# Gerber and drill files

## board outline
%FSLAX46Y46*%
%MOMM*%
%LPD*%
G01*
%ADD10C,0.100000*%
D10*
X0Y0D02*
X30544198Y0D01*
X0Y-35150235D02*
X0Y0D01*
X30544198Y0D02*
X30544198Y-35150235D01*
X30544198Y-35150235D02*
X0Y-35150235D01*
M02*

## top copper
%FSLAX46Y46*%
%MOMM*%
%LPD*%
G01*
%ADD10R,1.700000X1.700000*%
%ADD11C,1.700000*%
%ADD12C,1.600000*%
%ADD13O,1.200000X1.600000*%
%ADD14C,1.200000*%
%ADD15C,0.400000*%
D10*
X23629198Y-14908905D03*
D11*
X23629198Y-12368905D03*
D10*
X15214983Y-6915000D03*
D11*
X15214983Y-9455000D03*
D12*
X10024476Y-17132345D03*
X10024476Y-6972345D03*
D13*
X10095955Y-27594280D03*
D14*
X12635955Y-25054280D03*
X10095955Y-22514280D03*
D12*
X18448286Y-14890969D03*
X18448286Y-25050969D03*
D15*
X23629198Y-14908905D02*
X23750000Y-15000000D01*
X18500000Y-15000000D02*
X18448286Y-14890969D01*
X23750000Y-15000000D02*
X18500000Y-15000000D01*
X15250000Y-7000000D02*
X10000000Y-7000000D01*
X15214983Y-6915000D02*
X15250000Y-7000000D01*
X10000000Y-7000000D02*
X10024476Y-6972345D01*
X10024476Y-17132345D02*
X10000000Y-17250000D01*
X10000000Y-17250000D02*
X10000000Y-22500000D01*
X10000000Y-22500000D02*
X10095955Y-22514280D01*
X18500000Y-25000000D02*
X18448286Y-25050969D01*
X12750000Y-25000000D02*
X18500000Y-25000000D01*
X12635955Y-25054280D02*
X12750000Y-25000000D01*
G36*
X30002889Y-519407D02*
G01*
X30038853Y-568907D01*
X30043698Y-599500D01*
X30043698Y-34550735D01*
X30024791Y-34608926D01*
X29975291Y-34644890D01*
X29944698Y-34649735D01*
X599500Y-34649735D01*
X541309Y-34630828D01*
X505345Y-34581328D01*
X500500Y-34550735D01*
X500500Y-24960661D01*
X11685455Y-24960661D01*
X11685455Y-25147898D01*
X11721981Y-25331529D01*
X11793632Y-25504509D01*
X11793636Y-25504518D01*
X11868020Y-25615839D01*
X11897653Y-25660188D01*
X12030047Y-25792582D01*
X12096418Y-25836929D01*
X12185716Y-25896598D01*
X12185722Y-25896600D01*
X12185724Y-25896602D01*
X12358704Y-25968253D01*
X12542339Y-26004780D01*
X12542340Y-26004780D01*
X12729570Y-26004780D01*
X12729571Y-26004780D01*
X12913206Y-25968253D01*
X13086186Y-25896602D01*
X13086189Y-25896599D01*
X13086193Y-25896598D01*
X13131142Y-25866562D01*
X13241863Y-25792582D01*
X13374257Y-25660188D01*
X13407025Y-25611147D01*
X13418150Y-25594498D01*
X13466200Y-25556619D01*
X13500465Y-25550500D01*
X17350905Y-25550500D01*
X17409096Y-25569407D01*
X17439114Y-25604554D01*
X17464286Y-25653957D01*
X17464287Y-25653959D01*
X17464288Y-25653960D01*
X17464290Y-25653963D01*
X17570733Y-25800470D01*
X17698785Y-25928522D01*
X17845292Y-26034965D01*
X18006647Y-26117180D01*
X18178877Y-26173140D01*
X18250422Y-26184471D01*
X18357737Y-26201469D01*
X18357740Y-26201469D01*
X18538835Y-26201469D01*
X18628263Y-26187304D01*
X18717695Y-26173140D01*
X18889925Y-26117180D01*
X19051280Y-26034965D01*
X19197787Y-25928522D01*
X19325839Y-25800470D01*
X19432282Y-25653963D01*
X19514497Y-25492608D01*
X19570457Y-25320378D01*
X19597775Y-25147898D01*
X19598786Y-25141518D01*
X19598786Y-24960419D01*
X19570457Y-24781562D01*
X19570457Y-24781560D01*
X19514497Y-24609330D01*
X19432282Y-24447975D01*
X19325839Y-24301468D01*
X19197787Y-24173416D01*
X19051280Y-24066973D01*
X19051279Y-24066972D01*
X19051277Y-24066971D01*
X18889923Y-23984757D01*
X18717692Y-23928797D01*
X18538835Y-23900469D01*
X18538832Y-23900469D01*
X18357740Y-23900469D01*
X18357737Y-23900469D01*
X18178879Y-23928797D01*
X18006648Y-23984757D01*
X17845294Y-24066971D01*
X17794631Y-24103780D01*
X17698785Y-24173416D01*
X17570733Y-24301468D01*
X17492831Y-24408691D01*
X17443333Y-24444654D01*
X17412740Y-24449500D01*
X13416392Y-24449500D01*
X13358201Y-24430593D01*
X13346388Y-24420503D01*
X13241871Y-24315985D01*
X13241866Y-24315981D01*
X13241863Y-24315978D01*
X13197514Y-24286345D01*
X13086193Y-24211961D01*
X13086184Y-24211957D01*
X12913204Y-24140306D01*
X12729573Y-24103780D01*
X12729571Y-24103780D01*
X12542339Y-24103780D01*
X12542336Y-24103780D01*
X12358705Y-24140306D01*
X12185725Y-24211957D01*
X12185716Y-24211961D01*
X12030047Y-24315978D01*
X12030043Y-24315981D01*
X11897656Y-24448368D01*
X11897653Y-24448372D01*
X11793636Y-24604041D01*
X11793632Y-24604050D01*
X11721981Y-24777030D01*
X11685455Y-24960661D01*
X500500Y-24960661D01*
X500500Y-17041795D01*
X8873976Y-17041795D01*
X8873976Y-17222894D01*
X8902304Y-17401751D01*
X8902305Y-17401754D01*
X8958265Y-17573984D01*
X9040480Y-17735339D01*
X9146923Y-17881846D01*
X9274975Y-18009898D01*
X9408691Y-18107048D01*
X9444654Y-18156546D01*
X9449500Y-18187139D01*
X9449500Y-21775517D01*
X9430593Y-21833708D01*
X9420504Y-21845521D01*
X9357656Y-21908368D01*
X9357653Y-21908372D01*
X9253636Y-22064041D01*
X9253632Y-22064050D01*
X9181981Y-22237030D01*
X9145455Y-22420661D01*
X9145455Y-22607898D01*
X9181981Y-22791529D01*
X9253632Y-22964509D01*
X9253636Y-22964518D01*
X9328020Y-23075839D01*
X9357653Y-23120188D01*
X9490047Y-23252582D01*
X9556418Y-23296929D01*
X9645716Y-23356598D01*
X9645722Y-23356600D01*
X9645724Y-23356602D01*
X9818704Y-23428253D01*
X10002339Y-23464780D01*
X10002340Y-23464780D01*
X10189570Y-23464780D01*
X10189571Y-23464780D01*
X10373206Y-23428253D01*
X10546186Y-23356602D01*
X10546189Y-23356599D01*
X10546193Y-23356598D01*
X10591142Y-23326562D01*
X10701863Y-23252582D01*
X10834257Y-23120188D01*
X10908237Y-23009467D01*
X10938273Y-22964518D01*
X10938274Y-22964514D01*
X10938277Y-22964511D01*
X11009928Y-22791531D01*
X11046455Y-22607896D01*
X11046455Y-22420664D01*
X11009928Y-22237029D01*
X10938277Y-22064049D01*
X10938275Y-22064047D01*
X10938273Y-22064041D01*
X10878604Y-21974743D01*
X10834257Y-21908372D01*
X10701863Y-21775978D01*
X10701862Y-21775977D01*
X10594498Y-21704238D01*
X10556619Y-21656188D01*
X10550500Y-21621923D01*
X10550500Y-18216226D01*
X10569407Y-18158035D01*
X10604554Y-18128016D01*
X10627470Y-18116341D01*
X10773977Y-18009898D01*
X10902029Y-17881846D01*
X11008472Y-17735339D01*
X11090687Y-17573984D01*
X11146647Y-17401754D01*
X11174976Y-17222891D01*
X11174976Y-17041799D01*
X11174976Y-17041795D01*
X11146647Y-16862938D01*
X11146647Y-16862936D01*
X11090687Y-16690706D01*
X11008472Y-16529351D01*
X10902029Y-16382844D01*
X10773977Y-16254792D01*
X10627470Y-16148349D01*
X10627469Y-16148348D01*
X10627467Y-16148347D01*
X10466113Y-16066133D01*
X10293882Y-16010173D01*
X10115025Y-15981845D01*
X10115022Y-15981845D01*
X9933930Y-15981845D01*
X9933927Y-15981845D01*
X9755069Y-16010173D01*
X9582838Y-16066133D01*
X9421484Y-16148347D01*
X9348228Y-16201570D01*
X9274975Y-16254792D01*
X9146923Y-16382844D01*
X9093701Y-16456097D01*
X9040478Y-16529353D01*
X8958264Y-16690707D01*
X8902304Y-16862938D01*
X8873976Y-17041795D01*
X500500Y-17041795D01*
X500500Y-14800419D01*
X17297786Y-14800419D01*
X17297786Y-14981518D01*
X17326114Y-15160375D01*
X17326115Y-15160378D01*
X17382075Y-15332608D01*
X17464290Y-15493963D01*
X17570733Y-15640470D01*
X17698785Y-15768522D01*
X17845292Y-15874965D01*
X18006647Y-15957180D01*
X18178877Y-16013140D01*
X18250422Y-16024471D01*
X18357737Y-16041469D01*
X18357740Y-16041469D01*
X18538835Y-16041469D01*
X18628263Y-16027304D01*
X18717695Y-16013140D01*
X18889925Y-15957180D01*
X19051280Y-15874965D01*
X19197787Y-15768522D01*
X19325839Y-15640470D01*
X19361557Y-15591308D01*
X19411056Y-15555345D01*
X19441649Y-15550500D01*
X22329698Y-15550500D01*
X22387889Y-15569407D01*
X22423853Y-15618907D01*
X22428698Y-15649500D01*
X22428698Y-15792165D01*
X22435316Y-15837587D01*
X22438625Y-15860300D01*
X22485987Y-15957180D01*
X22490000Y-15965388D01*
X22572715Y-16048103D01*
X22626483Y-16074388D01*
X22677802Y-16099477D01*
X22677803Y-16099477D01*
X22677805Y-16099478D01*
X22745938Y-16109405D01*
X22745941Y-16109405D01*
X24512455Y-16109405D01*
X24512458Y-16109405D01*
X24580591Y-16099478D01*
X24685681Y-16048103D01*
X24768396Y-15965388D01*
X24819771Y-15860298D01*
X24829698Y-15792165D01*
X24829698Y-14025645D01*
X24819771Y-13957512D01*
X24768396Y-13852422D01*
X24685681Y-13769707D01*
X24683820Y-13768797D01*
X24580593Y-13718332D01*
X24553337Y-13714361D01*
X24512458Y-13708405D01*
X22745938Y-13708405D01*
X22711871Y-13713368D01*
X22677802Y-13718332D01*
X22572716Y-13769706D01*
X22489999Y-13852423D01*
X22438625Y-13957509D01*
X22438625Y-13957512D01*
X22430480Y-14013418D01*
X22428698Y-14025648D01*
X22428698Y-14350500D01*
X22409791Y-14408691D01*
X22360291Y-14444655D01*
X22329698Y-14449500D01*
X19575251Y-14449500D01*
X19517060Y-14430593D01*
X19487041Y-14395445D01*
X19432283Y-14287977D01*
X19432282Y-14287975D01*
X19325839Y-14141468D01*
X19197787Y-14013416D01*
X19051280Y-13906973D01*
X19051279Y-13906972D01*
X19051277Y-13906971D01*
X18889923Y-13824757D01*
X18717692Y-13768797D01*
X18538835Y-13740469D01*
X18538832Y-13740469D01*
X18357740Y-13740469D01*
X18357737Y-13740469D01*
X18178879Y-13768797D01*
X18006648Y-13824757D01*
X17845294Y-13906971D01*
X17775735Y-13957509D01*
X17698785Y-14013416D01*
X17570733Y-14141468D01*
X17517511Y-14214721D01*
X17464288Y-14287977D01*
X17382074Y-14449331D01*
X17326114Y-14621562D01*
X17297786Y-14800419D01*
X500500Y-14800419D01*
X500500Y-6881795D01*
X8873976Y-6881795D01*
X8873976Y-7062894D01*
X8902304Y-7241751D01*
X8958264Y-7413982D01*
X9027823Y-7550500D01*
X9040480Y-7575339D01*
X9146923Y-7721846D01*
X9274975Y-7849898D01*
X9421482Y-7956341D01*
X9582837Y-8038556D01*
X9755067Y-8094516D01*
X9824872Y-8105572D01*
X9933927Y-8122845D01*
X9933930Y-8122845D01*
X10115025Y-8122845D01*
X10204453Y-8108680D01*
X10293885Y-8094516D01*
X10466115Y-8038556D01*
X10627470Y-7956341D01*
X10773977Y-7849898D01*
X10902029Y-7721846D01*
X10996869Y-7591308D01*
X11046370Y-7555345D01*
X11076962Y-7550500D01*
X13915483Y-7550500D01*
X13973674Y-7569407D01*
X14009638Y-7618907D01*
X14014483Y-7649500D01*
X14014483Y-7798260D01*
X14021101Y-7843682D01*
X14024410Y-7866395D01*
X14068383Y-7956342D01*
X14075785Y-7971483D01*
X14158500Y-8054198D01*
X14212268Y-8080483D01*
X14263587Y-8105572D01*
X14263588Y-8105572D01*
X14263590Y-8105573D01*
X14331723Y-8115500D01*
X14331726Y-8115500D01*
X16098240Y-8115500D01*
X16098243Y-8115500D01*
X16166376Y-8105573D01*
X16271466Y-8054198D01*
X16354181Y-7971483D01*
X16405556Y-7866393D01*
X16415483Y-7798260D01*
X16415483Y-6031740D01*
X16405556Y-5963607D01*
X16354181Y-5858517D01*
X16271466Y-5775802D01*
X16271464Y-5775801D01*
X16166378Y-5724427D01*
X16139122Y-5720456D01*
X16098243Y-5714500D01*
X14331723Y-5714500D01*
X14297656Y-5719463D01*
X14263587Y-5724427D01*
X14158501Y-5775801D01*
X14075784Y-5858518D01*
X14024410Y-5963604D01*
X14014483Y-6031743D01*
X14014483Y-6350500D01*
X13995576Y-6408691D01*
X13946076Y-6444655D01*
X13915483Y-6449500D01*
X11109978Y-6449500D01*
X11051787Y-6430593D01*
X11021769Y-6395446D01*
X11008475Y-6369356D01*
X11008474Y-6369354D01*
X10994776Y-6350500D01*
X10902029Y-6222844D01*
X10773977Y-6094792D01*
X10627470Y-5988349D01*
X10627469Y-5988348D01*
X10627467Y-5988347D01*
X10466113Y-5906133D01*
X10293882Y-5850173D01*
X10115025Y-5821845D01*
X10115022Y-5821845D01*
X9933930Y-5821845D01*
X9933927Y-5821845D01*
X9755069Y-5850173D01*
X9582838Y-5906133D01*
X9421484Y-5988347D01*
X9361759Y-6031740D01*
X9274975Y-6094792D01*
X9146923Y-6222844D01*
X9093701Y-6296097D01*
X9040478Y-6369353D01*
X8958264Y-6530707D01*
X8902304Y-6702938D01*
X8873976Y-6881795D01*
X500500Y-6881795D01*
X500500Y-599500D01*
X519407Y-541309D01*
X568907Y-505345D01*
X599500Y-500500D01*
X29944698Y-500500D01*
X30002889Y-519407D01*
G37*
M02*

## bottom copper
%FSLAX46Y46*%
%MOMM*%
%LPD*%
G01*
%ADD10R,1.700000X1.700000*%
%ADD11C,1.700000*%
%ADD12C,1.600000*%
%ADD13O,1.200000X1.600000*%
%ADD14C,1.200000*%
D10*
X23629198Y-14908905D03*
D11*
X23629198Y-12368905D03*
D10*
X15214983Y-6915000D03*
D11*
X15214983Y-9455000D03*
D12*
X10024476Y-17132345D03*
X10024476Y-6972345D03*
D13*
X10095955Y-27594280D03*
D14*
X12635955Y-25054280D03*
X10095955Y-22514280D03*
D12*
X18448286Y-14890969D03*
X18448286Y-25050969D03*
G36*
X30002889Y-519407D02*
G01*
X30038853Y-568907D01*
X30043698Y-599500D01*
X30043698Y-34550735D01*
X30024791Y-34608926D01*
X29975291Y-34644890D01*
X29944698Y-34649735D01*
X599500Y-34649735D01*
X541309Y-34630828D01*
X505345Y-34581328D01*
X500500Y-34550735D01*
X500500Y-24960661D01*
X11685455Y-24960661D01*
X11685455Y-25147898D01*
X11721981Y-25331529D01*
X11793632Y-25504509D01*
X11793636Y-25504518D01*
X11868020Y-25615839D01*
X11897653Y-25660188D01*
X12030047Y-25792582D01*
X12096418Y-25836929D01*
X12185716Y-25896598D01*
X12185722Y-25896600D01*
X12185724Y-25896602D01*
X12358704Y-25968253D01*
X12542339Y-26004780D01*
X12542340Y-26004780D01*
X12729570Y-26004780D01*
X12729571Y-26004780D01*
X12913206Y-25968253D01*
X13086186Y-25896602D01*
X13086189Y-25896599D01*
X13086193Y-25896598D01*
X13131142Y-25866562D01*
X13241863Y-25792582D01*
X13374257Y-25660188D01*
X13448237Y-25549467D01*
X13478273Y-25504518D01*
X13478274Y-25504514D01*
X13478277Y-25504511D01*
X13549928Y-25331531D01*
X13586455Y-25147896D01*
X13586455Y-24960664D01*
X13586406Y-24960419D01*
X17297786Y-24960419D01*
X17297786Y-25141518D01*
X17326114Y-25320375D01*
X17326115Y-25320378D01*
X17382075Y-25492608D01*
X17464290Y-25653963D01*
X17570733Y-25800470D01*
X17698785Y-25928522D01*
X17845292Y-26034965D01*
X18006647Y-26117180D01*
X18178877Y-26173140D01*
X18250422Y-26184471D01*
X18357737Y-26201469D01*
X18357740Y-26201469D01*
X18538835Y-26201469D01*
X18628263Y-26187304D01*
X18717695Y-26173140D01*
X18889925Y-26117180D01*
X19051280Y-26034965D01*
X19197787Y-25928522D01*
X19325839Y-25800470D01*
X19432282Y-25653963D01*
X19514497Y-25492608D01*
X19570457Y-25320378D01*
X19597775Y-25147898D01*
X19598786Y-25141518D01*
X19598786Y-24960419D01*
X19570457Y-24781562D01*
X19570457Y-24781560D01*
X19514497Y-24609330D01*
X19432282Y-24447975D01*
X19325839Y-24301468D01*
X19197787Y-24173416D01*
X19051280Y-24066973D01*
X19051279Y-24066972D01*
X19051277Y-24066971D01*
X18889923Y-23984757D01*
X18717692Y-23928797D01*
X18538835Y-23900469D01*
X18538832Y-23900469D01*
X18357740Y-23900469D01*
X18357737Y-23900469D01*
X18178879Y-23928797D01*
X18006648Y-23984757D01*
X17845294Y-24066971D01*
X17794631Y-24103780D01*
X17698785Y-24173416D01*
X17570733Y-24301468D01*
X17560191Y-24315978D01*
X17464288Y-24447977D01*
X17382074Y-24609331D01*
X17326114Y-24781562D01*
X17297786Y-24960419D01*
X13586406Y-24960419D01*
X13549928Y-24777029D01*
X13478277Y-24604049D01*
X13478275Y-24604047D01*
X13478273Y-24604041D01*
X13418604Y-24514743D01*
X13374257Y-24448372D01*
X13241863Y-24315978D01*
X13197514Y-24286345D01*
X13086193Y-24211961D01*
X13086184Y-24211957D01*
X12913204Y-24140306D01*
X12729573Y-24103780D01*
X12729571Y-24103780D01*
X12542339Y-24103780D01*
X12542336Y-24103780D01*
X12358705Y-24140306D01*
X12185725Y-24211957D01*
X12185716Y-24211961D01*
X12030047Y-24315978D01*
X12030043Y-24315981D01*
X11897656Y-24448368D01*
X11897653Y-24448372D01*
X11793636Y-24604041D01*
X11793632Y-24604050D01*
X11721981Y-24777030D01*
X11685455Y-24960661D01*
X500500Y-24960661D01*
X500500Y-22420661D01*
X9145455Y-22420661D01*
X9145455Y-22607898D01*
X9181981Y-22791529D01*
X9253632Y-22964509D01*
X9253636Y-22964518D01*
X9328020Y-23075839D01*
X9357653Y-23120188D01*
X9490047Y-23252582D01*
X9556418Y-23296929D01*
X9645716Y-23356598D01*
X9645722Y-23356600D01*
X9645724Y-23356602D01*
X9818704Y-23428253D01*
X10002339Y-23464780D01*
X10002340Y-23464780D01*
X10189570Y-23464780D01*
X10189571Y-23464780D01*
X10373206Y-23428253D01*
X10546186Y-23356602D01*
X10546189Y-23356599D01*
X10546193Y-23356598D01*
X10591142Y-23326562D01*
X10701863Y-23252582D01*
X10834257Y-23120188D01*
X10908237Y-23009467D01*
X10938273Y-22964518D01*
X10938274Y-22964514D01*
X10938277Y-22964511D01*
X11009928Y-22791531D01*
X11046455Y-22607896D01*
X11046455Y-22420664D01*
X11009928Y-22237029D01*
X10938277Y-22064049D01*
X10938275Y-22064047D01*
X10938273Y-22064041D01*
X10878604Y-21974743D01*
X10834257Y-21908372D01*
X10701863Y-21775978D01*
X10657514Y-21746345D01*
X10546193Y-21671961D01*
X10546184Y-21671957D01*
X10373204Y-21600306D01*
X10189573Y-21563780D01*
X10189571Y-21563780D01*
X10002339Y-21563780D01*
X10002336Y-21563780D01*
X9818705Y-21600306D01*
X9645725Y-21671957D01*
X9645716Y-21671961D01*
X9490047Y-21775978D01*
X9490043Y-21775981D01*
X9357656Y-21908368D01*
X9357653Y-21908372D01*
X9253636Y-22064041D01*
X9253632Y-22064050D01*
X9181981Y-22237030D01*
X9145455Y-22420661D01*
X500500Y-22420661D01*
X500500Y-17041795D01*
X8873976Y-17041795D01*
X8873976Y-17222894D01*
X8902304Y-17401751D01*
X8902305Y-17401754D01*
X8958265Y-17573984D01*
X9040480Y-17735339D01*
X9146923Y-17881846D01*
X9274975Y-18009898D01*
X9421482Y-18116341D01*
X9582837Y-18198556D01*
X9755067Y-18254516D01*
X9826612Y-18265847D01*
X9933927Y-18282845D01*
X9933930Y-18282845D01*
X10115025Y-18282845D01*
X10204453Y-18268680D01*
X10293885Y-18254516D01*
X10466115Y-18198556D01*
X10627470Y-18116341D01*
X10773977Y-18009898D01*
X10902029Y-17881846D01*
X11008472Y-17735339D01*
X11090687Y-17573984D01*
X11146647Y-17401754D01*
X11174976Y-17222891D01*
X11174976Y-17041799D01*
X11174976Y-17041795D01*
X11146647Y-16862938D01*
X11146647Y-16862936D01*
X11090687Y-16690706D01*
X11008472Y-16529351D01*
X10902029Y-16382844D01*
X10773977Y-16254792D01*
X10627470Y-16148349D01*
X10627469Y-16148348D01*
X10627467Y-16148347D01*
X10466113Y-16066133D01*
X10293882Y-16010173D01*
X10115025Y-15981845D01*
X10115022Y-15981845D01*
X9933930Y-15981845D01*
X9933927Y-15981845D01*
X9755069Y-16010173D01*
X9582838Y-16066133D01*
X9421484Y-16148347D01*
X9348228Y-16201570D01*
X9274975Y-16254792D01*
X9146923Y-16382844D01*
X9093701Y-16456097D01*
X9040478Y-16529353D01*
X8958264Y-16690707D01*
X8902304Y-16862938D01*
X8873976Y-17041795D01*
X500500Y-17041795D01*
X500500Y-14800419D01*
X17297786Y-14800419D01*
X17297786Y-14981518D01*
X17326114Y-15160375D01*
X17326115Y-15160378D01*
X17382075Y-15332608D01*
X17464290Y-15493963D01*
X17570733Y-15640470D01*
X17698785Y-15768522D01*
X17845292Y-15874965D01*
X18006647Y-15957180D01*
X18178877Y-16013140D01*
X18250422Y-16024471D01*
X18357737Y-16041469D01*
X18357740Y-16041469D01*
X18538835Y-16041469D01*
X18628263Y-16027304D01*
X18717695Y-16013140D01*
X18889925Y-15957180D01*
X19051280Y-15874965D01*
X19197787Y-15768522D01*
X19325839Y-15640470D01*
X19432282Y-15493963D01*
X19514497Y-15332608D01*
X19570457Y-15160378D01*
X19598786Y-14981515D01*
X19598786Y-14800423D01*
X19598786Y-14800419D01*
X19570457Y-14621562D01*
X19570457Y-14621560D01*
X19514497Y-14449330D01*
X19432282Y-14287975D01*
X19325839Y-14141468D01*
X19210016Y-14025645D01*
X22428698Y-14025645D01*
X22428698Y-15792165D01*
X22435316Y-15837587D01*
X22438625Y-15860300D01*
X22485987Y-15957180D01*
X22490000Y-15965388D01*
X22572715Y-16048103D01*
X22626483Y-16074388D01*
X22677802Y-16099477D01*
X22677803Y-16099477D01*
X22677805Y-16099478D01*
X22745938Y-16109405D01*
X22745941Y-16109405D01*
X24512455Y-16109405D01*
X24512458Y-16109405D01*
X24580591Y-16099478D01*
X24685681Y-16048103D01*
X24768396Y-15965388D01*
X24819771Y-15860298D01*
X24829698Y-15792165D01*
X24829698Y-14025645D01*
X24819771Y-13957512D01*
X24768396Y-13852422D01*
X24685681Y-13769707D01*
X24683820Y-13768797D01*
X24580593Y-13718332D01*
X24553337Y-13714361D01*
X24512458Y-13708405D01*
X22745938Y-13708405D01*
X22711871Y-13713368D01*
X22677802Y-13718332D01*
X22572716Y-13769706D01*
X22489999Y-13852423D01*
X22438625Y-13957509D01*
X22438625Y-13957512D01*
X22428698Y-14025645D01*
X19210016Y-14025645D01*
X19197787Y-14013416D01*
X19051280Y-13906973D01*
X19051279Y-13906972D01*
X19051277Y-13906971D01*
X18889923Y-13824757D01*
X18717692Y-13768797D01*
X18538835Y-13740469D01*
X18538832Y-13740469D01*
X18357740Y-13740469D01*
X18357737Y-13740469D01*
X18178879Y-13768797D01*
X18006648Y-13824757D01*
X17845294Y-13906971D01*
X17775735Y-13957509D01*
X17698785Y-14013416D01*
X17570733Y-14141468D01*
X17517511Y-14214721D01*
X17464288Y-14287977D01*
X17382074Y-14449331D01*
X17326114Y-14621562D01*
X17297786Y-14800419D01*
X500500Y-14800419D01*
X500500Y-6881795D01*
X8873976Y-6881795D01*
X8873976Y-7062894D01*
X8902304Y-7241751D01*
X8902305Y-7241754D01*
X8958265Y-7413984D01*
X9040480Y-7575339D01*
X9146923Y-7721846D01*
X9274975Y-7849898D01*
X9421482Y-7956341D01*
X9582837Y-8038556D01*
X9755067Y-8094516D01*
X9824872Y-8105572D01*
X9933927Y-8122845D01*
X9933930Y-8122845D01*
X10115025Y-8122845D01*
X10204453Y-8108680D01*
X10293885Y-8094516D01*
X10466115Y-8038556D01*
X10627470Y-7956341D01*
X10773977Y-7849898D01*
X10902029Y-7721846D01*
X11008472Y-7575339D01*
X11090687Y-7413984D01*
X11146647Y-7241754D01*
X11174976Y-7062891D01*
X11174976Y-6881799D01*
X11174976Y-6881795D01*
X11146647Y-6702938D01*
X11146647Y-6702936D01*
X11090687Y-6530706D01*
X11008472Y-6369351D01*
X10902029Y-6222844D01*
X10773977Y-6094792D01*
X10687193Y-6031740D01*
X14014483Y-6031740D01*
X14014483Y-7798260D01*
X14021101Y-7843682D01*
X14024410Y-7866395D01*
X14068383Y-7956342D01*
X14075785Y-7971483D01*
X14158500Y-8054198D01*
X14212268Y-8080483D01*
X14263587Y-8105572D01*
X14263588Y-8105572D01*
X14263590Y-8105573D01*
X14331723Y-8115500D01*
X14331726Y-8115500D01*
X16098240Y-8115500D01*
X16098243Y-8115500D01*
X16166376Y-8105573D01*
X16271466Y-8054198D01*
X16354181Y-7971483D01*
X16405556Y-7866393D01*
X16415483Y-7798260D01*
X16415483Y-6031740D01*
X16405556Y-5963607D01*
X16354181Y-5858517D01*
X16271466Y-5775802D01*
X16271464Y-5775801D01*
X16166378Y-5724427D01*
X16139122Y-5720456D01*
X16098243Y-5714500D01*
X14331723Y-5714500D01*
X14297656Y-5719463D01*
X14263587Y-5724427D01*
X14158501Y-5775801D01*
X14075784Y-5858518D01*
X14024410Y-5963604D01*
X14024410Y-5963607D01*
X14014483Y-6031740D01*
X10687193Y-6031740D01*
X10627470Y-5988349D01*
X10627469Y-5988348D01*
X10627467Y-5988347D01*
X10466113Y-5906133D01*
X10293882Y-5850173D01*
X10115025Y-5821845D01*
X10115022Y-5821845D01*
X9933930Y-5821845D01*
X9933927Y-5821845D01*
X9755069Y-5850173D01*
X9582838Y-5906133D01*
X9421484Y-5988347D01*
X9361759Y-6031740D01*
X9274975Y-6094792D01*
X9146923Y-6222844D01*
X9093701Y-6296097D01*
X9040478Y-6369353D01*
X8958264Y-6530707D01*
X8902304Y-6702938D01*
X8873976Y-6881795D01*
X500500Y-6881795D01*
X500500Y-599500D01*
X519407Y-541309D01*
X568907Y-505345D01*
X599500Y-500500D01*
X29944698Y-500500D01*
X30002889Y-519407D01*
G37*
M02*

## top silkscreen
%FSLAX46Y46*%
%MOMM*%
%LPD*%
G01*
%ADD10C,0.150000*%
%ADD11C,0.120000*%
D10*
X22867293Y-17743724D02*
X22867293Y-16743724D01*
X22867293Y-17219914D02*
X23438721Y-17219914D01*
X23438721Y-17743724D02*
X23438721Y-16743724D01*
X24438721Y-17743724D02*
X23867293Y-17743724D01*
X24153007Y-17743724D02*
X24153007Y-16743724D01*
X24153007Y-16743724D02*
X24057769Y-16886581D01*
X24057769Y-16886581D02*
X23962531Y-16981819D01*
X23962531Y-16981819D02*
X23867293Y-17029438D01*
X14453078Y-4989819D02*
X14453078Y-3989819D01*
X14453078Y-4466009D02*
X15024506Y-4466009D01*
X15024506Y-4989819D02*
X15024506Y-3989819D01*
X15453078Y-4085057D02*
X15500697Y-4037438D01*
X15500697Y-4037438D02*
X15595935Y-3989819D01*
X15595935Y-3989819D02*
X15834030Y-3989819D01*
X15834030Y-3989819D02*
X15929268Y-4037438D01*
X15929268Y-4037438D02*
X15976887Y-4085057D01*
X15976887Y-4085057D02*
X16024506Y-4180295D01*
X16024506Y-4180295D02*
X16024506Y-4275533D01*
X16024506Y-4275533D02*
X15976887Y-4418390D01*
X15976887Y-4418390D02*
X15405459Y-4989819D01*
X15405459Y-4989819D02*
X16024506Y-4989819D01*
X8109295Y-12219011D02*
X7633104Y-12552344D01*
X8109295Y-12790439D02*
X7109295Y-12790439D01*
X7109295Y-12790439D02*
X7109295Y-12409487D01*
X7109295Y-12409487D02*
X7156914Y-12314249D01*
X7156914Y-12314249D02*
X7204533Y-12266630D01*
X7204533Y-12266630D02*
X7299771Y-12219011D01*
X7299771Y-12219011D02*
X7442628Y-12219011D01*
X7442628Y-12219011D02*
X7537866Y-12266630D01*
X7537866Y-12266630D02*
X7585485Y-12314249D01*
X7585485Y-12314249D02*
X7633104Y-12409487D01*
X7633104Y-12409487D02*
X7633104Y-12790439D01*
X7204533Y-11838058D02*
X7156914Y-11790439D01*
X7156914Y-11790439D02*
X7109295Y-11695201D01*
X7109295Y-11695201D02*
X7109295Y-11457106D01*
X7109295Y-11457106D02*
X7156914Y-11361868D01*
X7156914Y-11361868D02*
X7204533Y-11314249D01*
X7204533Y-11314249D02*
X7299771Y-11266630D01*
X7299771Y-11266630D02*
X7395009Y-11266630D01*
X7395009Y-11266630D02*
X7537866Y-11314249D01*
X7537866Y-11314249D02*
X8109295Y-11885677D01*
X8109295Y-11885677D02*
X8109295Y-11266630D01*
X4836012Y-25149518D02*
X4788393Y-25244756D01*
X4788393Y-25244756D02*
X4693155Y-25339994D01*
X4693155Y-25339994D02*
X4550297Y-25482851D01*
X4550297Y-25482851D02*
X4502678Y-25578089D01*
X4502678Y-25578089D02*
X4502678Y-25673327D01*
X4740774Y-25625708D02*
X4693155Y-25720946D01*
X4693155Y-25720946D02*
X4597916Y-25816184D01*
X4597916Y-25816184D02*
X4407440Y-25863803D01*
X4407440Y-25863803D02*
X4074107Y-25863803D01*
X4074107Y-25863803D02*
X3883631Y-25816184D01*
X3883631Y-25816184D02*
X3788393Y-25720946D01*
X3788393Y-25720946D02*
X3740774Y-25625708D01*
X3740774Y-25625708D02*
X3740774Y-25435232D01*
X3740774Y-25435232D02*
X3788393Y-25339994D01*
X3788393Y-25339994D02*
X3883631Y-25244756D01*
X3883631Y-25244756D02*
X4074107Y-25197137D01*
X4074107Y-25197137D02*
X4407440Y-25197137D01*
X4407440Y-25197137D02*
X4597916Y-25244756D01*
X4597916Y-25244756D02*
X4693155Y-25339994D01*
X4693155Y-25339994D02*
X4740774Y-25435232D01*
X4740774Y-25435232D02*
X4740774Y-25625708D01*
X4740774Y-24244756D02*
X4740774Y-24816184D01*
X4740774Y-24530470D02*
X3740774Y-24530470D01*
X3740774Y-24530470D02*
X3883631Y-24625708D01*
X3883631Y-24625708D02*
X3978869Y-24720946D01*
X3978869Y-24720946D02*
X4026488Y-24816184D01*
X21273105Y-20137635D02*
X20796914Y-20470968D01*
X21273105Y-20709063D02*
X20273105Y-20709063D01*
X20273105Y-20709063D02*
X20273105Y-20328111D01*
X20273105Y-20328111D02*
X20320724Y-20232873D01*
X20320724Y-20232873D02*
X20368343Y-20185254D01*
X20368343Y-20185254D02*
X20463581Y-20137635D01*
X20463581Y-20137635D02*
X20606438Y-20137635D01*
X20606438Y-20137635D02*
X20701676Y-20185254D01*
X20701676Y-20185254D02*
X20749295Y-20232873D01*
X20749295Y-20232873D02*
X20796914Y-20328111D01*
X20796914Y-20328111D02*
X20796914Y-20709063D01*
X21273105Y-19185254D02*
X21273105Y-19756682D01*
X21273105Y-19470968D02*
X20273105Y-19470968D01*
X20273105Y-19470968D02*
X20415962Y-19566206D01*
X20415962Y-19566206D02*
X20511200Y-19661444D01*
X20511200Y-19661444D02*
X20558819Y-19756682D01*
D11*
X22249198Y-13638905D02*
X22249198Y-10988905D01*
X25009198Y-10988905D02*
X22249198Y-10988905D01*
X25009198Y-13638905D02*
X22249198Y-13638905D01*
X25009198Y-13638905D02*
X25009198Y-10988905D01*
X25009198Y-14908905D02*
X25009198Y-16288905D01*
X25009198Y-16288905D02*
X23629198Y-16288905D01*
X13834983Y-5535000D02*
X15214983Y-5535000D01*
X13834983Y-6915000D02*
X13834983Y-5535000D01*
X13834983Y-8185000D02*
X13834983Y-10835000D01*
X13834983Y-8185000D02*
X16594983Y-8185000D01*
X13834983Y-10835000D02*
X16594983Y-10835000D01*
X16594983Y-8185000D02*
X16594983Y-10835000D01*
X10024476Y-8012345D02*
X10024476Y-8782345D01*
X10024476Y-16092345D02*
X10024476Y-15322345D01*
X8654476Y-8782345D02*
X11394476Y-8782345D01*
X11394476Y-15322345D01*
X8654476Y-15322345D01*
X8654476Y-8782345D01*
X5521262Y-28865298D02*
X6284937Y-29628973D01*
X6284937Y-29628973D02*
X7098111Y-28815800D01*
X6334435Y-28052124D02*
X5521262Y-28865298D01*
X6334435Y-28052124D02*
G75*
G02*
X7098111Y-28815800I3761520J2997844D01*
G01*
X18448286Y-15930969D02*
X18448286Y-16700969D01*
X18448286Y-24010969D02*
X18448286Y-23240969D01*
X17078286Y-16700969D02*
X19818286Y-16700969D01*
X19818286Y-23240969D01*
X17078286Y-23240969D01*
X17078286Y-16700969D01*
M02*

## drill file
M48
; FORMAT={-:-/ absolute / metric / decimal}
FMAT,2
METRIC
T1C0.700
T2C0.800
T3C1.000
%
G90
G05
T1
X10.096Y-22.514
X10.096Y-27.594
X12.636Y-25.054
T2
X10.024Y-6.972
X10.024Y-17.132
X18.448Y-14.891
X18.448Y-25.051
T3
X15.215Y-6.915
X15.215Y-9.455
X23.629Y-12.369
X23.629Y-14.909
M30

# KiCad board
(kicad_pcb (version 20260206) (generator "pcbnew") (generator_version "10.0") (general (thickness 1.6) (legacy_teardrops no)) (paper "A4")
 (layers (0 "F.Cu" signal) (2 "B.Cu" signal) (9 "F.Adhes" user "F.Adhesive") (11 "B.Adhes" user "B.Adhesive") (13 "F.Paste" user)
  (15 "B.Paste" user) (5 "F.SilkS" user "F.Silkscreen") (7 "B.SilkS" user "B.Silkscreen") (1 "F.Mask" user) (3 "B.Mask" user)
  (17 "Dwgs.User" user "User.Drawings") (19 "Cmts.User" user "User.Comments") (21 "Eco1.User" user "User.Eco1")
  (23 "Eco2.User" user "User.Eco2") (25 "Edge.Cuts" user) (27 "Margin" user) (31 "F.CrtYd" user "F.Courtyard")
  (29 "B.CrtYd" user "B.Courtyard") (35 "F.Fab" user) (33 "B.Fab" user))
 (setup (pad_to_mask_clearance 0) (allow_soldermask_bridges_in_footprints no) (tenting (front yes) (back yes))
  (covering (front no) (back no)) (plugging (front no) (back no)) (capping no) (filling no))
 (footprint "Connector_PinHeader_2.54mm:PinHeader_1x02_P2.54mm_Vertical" (layer "F.Cu") (at 23.629198 14.908905 180)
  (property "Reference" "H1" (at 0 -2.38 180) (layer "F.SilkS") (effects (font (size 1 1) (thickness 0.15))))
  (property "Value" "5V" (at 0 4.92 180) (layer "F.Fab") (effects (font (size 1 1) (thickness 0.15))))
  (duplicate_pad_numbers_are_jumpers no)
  (fp_line (start 1.38 1.27) (end 1.38 3.92) (stroke (width 0.12) (type solid)) (layer "F.SilkS"))
  (fp_line (start -1.38 3.92) (end 1.38 3.92) (stroke (width 0.12) (type solid)) (layer "F.SilkS"))
  (fp_line (start -1.38 1.27) (end 1.38 1.27) (stroke (width 0.12) (type solid)) (layer "F.SilkS"))
  (fp_line (start -1.38 1.27) (end -1.38 3.92) (stroke (width 0.12) (type solid)) (layer "F.SilkS"))
  (fp_line (start -1.38 0) (end -1.38 -1.38) (stroke (width 0.12) (type solid)) (layer "F.SilkS"))
  (fp_line (start -1.38 -1.38) (end 0 -1.38) (stroke (width 0.12) (type solid)) (layer "F.SilkS"))
  (pad "1" thru_hole rect (at 0 0 180) (size 1.7 1.7) (drill 1) (layers "*.Cu" "*.Mask") (remove_unused_layers no) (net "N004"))
  (pad "2" thru_hole circle (at 0 2.54 180) (size 1.7 1.7) (drill 1) (layers "*.Cu" "*.Mask") (remove_unused_layers no) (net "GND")))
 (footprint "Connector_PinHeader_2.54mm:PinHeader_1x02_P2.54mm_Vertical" (layer "F.Cu") (at 15.214983 6.915)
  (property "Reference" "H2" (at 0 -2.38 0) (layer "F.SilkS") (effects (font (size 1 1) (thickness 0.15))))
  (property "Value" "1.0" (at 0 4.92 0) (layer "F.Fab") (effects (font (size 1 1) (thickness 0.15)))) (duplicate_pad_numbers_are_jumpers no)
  (fp_line (start -1.38 -1.38) (end 0 -1.38) (stroke (width 0.12) (type solid)) (layer "F.SilkS"))
  (fp_line (start -1.38 0) (end -1.38 -1.38) (stroke (width 0.12) (type solid)) (layer "F.SilkS"))
  (fp_line (start -1.38 1.27) (end -1.38 3.92) (stroke (width 0.12) (type solid)) (layer "F.SilkS"))
  (fp_line (start -1.38 1.27) (end 1.38 1.27) (stroke (width 0.12) (type solid)) (layer "F.SilkS"))
  (fp_line (start -1.38 3.92) (end 1.38 3.92) (stroke (width 0.12) (type solid)) (layer "F.SilkS"))
  (fp_line (start 1.38 1.27) (end 1.38 3.92) (stroke (width 0.12) (type solid)) (layer "F.SilkS"))
  (pad "1" thru_hole rect (at 0 0) (size 1.7 1.7) (drill 1) (layers "*.Cu" "*.Mask") (remove_unused_layers no) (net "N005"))
  (pad "2" thru_hole circle (at 0 2.54) (size 1.7 1.7) (drill 1) (layers "*.Cu" "*.Mask") (remove_unused_layers no) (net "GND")))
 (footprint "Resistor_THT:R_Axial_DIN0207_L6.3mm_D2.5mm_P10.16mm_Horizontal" (layer "F.Cu") (at 10.024476 17.132345 90)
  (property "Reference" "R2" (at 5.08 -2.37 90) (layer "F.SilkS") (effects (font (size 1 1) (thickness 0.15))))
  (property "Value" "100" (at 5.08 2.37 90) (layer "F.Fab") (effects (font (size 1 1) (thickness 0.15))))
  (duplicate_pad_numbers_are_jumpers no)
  (fp_line (start 9.12 0) (end 8.35 0) (stroke (width 0.12) (type solid)) (layer "F.SilkS"))
  (fp_line (start 1.04 0) (end 1.81 0) (stroke (width 0.12) (type solid)) (layer "F.SilkS"))
  (fp_rect (start 1.81 -1.37) (end 8.35 1.37) (stroke (width 0.12) (type solid)) (fill no) (layer "F.SilkS"))
  (pad "1" thru_hole circle (at 0 0 90) (size 1.6 1.6) (drill 0.8) (layers "*.Cu" "*.Mask") (remove_unused_layers no) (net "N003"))
  (pad "2" thru_hole circle (at 10.16 0 90) (size 1.6 1.6) (drill 0.8) (layers "*.Cu" "*.Mask") (remove_unused_layers no) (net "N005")))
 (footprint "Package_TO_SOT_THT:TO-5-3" (layer "F.Cu") (at 10.095955 27.59428 90)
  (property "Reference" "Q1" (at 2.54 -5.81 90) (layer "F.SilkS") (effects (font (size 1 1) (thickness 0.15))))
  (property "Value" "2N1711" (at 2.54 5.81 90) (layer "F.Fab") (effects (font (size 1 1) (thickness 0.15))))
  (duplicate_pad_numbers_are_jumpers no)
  (fp_line (start -1.271018 -4.574693) (end -2.034693 -3.811018) (stroke (width 0.12) (type solid)) (layer "F.SilkS"))
  (fp_line (start -2.034693 -3.811018) (end -1.22152 -2.997844) (stroke (width 0.12) (type solid)) (layer "F.SilkS"))
  (fp_line (start -0.457844 -3.76152) (end -1.271018 -4.574693) (stroke (width 0.12) (type solid)) (layer "F.SilkS"))
  (fp_arc (start -0.457844 -3.76152) (mid 5.941184 3.401184) (end -1.22152 -2.997844) (stroke (width 0.12) (type solid)) (layer "F.SilkS"))
  (pad "1" thru_hole oval (at 0 0 90) (size 1.6 1.2) (drill 0.7) (layers "*.Cu" "*.Mask") (remove_unused_layers no) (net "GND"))
  (pad "2" thru_hole circle (at 2.54 2.54 90) (size 1.2 1.2) (drill 0.7) (layers "*.Cu" "*.Mask") (remove_unused_layers no) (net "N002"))
  (pad "3" thru_hole circle (at 5.08 0 90) (size 1.2 1.2) (drill 0.7) (layers "*.Cu" "*.Mask") (remove_unused_layers no) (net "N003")))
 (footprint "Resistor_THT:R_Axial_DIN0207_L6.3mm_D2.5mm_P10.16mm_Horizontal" (layer "F.Cu") (at 18.448286 14.890969 -90)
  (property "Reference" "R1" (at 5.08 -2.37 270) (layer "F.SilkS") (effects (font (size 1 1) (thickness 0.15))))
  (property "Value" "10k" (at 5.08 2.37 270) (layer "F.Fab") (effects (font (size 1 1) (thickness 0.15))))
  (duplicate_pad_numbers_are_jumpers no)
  (fp_line (start 1.04 0) (end 1.81 0) (stroke (width 0.12) (type solid)) (layer "F.SilkS"))
  (fp_line (start 9.12 0) (end 8.35 0) (stroke (width 0.12) (type solid)) (layer "F.SilkS"))
  (fp_rect (start 1.81 -1.37) (end 8.35 1.37) (stroke (width 0.12) (type solid)) (fill no) (layer "F.SilkS"))
  (pad "1" thru_hole circle (at 0 0 270) (size 1.6 1.6) (drill 0.8) (layers "*.Cu" "*.Mask") (remove_unused_layers no) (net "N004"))
  (pad "2" thru_hole circle (at 10.16 0 270) (size 1.6 1.6) (drill 0.8) (layers "*.Cu" "*.Mask") (remove_unused_layers no) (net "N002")))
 (gr_line (start 0 0) (end 30.544198 0) (stroke (width 0.1) (type default)) (layer "Edge.Cuts"))
 (gr_line (start 0 35.150235) (end 0 0) (stroke (width 0.1) (type default)) (layer "Edge.Cuts"))
 (gr_line (start 30.544198 0) (end 30.544198 35.150235) (stroke (width 0.1) (type default)) (layer "Edge.Cuts"))
 (gr_line (start 30.544198 35.150235) (end 0 35.150235) (stroke (width 0.1) (type default)) (layer "Edge.Cuts"))
 (segment (start 23.629198 14.908905) (end 23.75 15) (width 0.4) (layer "F.Cu") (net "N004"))
 (segment (start 18.5 15) (end 18.448286 14.890969) (width 0.4) (layer "F.Cu") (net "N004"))
 (segment (start 23.75 15) (end 18.5 15) (width 0.4) (layer "F.Cu") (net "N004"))
 (segment (start 15.25 7) (end 10 7) (width 0.4) (layer "F.Cu") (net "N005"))
 (segment (start 15.214983 6.915) (end 15.25 7) (width 0.4) (layer "F.Cu") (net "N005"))
 (segment (start 10 7) (end 10.024476 6.972345) (width 0.4) (layer "F.Cu") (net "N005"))
 (segment (start 10.024476 17.132345) (end 10 17.25) (width 0.4) (layer "F.Cu") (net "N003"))
 (segment (start 10 17.25) (end 10 22.5) (width 0.4) (layer "F.Cu") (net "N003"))
 (segment (start 10 22.5) (end 10.095955 22.51428) (width 0.4) (layer "F.Cu") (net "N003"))
 (segment (start 18.5 25) (end 18.448286 25.050969) (width 0.4) (layer "F.Cu") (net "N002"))
 (segment (start 12.75 25) (end 18.5 25) (width 0.4) (layer "F.Cu") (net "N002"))
 (segment (start 12.635955 25.05428) (end 12.75 25) (width 0.4) (layer "F.Cu") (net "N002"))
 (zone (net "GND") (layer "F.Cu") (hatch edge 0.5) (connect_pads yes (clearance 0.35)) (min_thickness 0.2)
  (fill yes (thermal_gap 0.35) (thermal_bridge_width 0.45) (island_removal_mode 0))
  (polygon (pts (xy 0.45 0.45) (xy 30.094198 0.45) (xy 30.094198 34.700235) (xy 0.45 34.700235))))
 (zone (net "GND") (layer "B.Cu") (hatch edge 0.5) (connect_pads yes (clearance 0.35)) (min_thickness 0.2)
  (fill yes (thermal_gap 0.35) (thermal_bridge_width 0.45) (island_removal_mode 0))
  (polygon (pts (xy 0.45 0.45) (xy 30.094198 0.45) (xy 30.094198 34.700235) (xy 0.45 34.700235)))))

